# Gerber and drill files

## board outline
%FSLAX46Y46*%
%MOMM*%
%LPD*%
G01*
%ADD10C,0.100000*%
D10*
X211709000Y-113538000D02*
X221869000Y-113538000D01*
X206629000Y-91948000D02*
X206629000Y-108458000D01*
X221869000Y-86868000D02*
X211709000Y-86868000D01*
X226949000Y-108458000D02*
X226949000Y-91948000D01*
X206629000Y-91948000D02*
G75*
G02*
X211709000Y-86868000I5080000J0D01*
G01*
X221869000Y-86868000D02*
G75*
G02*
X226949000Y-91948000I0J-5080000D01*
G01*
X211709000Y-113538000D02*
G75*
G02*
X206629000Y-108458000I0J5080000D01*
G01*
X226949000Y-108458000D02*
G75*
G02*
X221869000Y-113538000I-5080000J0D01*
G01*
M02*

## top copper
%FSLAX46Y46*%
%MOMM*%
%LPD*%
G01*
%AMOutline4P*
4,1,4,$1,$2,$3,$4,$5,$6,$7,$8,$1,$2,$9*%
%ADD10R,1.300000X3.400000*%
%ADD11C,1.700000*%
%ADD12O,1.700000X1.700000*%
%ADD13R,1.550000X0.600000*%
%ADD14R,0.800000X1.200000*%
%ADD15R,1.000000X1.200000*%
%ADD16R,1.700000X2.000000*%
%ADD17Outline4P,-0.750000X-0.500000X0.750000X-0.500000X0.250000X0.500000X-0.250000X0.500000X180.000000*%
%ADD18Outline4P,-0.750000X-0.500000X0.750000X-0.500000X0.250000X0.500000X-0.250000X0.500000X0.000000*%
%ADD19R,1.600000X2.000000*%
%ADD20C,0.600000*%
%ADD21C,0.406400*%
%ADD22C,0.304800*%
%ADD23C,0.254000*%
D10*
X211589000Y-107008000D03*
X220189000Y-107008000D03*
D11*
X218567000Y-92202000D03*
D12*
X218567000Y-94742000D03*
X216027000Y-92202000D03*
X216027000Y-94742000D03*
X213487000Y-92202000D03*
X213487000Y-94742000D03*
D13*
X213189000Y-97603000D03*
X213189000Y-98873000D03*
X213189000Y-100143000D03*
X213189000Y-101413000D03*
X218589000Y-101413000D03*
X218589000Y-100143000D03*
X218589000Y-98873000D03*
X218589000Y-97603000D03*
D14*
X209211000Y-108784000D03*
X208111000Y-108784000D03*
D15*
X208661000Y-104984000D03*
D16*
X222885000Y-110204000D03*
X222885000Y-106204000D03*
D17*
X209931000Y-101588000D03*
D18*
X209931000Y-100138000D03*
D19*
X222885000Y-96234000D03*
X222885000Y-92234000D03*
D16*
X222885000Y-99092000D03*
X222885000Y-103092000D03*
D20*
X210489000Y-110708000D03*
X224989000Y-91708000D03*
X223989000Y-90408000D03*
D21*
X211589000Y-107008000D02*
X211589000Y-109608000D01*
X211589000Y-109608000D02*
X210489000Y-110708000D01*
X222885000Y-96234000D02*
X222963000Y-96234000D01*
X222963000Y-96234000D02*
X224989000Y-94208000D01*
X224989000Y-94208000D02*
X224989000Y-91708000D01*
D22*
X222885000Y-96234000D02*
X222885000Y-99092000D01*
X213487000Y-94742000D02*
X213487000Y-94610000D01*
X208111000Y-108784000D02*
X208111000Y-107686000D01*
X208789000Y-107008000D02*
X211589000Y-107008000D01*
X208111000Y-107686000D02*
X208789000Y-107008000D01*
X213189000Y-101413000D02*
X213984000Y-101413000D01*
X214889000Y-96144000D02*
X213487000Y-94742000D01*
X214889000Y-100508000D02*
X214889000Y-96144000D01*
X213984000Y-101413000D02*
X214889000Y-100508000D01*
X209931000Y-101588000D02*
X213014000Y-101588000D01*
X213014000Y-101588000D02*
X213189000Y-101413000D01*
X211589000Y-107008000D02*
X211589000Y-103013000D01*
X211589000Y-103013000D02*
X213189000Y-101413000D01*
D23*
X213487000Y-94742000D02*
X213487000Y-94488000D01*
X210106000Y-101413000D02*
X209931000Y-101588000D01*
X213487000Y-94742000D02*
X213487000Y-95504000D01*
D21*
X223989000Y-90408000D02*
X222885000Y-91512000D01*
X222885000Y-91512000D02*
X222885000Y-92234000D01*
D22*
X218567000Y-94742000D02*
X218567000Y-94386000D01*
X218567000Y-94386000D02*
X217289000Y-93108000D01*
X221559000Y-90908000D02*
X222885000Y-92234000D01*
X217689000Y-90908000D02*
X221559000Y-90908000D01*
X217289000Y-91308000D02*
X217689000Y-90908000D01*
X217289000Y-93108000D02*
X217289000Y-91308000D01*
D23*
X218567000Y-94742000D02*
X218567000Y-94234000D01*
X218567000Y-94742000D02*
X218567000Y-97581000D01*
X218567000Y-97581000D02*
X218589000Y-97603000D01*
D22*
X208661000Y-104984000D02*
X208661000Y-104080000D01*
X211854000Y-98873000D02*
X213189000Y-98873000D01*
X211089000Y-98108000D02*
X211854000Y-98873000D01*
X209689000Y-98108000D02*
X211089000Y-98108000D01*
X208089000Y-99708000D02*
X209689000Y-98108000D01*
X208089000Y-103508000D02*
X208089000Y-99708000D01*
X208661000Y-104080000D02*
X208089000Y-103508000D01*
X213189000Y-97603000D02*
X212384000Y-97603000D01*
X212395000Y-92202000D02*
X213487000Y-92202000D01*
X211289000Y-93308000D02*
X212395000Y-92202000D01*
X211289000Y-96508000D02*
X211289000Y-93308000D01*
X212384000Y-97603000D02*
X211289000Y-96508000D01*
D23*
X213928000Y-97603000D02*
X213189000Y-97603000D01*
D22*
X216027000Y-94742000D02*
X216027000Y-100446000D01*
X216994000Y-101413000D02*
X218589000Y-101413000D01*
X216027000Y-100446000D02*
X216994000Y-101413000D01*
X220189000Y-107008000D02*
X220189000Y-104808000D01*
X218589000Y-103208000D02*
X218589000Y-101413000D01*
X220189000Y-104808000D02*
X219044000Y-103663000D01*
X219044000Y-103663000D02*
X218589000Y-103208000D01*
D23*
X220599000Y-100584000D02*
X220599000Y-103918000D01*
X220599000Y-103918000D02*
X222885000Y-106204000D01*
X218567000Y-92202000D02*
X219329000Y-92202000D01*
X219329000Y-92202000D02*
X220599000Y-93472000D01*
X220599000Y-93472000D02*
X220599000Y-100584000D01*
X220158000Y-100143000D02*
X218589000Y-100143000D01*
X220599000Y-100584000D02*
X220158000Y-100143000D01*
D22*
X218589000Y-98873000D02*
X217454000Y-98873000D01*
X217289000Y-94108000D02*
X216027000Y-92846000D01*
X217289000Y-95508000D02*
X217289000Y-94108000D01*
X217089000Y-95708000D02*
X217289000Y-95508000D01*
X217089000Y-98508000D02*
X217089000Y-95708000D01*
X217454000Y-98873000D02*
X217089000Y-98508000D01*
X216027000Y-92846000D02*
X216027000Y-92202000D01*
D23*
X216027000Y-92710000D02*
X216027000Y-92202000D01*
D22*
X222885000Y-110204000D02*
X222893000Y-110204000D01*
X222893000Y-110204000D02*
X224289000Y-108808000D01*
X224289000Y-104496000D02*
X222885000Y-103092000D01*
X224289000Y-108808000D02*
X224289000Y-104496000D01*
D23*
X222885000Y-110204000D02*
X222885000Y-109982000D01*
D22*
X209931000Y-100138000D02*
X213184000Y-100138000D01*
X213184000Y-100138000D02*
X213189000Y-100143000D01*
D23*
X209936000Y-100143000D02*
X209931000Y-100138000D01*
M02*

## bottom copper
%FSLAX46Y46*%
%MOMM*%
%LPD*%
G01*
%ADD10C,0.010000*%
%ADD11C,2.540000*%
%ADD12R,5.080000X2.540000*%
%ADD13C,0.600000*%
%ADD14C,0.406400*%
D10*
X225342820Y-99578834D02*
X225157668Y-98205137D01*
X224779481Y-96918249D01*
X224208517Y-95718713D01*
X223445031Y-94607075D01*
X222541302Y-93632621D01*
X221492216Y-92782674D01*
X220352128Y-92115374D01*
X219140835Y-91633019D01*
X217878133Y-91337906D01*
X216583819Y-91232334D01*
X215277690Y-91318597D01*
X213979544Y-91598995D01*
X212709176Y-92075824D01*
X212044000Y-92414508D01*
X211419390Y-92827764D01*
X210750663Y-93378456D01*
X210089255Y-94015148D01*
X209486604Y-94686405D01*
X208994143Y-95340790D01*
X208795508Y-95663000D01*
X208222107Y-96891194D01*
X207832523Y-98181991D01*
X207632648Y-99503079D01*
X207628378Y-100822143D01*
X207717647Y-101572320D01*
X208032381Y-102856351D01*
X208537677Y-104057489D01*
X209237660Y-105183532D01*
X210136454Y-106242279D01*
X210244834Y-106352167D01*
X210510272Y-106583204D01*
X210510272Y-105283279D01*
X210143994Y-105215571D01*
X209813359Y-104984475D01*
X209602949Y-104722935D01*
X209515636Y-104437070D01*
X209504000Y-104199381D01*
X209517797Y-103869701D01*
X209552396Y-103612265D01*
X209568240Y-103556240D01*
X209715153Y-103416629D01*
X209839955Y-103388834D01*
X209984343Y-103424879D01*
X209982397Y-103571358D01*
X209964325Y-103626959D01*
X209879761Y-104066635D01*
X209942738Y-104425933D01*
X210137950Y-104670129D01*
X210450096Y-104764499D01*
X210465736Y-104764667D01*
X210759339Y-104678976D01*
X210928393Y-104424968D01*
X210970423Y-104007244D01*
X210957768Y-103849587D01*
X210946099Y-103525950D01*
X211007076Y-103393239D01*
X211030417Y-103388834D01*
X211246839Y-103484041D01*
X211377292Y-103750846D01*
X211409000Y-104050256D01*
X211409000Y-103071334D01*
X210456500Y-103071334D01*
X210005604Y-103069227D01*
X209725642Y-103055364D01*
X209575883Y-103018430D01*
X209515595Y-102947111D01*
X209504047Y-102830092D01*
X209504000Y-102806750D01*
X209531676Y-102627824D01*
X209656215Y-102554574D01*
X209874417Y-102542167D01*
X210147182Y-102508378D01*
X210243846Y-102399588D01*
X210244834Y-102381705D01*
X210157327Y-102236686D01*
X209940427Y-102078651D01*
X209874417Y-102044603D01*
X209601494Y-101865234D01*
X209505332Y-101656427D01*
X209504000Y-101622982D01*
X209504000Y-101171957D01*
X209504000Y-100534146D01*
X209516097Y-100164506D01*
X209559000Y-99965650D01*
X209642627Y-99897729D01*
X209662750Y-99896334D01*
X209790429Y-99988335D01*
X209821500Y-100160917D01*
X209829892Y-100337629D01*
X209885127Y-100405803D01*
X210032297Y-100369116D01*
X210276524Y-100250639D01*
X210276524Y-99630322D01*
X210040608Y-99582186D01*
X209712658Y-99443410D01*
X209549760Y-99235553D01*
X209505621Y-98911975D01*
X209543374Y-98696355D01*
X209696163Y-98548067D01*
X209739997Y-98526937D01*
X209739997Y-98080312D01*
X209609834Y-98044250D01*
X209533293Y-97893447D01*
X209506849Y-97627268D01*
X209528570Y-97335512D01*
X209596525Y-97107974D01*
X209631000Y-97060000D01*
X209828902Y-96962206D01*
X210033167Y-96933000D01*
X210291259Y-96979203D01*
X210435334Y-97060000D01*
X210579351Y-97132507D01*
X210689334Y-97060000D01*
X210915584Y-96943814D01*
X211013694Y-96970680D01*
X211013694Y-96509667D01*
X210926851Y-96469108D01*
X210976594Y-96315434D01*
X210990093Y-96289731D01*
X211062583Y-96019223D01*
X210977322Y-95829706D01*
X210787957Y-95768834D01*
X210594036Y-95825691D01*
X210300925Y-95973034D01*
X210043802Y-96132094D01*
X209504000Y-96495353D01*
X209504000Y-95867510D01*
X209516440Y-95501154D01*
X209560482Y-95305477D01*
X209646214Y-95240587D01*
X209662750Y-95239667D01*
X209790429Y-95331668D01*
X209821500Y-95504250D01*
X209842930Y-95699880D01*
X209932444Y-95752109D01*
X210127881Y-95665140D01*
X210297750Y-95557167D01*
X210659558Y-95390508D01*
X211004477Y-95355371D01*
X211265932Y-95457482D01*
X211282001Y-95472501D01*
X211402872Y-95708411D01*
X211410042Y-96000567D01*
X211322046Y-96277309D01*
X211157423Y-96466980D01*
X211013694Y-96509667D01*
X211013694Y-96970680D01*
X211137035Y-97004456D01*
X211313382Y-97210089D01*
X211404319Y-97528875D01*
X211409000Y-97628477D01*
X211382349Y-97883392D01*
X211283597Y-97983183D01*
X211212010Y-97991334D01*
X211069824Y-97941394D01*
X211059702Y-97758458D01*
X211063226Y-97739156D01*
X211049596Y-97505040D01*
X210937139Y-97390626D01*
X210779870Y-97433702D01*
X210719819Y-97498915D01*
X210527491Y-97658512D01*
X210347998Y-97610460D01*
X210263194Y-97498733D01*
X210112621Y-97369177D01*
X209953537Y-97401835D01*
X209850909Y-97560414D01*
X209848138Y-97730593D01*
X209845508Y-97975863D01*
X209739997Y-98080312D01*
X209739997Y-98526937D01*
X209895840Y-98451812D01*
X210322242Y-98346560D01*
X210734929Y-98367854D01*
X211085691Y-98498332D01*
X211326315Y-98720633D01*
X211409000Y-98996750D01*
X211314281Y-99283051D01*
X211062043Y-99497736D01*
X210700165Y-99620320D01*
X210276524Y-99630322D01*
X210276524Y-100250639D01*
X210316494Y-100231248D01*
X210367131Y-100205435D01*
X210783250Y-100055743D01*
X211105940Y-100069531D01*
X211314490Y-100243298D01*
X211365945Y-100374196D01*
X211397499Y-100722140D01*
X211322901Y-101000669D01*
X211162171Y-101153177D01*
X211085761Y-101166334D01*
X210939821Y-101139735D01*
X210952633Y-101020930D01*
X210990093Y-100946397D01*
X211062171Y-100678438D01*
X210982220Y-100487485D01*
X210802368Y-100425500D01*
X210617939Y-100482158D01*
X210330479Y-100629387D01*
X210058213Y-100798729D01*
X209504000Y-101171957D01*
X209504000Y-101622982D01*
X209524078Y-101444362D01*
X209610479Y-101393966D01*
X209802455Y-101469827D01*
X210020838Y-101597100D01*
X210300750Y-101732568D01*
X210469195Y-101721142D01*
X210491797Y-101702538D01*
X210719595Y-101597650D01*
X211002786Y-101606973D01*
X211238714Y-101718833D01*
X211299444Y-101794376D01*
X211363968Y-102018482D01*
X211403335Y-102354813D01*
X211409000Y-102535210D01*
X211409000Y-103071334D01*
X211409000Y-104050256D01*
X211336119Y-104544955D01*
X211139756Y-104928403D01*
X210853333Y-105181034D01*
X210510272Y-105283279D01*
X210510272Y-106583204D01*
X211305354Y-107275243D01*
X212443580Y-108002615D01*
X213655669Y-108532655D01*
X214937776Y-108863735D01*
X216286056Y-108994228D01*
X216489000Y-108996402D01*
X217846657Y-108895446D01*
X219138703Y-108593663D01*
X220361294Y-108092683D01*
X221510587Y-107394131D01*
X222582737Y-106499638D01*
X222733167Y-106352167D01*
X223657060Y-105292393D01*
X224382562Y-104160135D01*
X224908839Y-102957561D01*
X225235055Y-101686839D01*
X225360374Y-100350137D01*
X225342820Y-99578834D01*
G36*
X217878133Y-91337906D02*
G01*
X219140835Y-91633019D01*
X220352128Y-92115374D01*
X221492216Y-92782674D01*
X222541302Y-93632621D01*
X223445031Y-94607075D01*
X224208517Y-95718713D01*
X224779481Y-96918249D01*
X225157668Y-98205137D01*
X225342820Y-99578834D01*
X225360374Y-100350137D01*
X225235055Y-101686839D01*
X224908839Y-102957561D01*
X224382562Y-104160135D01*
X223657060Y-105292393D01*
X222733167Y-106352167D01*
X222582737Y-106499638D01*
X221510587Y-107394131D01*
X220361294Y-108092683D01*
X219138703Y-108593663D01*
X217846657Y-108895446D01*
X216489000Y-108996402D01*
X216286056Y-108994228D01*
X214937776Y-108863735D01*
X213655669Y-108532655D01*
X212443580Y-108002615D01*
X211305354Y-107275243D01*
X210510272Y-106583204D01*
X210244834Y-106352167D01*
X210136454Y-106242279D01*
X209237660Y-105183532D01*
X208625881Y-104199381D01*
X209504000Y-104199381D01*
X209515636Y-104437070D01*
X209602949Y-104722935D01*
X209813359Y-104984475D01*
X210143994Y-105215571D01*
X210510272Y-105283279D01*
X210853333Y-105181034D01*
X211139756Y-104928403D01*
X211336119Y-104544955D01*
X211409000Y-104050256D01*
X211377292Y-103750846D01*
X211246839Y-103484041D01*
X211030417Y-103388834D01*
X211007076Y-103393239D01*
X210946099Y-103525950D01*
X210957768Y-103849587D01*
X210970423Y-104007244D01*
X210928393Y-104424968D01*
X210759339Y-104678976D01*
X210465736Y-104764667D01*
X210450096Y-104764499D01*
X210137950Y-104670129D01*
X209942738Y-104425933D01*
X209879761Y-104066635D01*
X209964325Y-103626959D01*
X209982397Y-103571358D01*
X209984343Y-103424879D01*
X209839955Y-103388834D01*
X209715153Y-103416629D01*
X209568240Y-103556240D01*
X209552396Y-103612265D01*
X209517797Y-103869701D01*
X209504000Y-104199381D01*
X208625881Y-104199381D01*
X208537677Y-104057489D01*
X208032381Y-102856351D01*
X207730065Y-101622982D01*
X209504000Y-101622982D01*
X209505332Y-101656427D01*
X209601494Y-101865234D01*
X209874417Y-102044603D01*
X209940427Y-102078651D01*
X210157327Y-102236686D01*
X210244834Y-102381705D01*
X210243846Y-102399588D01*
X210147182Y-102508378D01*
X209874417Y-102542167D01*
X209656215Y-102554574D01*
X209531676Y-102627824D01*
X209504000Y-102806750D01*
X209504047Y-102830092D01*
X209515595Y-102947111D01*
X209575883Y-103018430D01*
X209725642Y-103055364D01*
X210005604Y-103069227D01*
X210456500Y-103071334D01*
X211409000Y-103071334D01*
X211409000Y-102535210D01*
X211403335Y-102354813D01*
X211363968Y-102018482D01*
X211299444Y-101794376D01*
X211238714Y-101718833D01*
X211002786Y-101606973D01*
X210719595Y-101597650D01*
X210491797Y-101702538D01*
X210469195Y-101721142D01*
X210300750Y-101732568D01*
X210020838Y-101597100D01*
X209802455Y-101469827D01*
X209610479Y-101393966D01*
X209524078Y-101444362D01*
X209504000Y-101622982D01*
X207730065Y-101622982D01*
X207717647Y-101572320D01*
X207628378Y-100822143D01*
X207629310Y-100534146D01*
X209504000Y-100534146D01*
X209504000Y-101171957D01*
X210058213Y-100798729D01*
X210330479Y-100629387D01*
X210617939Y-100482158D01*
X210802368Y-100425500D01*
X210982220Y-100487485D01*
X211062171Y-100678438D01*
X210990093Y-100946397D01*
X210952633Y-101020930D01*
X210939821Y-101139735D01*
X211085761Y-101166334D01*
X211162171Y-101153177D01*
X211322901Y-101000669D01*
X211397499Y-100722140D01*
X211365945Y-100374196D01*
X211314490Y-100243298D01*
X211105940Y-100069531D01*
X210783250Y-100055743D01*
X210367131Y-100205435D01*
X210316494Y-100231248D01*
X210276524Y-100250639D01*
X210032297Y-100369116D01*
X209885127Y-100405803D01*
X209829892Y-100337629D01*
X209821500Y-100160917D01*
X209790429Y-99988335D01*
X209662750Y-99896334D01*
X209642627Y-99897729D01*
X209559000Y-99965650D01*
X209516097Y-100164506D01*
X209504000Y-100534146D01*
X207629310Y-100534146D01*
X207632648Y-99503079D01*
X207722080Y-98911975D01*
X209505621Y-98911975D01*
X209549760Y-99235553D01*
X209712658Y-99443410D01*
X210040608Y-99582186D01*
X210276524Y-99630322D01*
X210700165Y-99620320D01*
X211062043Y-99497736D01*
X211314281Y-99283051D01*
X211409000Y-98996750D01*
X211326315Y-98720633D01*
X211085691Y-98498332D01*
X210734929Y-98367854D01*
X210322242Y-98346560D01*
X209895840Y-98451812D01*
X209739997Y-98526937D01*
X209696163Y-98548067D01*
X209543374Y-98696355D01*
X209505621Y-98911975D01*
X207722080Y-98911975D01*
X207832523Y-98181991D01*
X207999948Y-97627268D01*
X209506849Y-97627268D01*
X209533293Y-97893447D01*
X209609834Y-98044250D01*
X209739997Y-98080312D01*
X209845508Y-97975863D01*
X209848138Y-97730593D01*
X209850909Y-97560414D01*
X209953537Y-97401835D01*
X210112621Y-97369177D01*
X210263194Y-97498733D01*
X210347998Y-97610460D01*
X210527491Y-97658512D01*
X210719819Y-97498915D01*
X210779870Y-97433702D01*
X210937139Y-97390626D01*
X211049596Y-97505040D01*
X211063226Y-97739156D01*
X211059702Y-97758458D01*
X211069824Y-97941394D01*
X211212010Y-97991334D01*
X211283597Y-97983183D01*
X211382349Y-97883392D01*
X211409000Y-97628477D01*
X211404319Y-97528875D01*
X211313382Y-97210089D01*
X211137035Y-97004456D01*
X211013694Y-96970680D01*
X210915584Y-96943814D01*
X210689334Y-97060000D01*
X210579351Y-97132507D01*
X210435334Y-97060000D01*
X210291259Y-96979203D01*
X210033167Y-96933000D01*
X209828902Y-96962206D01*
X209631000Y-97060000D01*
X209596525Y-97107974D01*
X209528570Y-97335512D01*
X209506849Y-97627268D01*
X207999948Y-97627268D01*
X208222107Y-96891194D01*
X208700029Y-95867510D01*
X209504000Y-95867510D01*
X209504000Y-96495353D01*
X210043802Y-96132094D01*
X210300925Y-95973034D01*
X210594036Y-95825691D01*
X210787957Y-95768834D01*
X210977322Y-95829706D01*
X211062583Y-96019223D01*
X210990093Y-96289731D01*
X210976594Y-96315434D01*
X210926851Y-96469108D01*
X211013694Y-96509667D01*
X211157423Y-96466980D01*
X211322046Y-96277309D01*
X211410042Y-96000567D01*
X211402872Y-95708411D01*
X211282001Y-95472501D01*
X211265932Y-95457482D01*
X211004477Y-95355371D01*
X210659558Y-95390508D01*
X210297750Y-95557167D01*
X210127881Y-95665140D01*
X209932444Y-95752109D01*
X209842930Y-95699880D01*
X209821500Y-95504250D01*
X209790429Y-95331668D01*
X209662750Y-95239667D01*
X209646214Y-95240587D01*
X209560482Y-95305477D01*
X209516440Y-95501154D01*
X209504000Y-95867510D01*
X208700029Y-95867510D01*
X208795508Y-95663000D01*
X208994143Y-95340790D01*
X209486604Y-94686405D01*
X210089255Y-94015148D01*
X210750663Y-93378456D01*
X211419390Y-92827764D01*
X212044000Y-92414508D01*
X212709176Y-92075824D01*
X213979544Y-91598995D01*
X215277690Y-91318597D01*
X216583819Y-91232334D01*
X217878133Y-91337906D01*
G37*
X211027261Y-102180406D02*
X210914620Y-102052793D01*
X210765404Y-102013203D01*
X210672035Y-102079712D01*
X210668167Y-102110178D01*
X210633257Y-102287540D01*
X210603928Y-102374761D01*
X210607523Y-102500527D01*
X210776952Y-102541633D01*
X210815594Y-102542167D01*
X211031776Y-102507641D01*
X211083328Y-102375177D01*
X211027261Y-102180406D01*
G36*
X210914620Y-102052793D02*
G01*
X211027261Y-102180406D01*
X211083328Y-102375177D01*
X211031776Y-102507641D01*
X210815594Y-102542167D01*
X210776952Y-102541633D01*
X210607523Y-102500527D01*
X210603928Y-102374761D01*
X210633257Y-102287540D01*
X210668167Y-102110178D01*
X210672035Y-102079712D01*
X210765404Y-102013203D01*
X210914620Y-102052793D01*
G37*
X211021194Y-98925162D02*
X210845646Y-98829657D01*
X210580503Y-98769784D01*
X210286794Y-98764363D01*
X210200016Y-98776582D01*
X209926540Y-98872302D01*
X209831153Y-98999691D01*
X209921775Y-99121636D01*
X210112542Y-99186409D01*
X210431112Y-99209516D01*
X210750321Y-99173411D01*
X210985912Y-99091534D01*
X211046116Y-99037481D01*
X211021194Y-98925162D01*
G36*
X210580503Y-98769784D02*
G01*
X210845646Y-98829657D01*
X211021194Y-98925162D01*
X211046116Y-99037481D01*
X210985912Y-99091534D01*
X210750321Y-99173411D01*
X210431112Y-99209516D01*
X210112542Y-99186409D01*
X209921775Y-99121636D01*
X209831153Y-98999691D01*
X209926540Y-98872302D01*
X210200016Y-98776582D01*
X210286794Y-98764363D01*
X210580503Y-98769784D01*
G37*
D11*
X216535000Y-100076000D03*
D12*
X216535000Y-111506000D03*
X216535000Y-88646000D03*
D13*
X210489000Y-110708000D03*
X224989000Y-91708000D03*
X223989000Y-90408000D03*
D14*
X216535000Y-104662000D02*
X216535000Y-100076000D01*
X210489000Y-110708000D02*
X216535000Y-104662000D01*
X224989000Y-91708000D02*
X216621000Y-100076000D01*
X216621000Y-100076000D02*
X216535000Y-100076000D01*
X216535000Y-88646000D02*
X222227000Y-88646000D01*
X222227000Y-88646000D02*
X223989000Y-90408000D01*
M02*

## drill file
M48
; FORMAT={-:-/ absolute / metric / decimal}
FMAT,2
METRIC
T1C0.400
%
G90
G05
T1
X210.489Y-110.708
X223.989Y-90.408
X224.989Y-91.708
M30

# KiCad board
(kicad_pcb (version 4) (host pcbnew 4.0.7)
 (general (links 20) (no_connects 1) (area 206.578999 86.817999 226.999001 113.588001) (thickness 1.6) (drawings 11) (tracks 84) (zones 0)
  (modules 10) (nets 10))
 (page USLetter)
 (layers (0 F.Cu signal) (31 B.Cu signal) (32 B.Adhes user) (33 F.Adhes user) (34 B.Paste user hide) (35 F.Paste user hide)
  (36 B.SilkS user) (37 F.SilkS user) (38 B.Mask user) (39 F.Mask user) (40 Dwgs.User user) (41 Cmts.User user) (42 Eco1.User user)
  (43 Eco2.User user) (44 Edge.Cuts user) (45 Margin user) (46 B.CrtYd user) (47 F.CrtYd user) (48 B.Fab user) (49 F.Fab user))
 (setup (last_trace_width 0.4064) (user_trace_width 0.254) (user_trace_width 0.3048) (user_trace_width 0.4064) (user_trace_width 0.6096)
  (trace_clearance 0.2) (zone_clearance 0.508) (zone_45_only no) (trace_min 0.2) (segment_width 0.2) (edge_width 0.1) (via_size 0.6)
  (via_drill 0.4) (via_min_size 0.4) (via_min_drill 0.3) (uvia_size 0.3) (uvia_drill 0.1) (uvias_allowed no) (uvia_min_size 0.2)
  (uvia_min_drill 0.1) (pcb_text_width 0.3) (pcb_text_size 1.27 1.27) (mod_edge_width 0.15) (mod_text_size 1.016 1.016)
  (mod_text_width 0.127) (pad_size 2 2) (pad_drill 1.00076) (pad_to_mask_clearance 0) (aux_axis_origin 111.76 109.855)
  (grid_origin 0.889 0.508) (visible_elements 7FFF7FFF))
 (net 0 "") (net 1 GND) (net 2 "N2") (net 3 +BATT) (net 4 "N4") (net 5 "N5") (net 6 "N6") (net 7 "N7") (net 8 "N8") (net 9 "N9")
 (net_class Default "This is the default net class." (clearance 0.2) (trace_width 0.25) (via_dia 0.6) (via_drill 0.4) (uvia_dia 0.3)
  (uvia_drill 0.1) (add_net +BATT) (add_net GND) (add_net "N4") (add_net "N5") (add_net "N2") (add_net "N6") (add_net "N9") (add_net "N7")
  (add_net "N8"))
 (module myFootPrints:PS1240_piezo (layer F.Cu) (at 215.889 107.008)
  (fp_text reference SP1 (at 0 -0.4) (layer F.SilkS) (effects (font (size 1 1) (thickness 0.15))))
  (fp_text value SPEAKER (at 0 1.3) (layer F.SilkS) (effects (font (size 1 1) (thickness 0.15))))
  (pad 1 smd rect (at -4.3 0) (size 1.3 3.4) (layers F.Cu F.Paste F.Mask) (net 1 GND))
  (pad 2 smd rect (at 4.3 0) (size 1.3 3.4) (layers F.Cu F.Paste F.Mask) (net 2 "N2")))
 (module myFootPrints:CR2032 (layer B.Cu) (at 216.489 100.108 90)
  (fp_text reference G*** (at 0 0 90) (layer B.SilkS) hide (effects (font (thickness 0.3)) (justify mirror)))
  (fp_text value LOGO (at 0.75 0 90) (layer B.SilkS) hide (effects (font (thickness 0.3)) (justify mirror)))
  (fp_poly
   (pts (xy 0.529166 8.85382) (xy 1.902863 8.668668) (xy 3.189751 8.290481) (xy 4.389287 7.719517) (xy 5.500925 6.956031)
    (xy 6.475379 6.052302) (xy 7.325326 5.003216) (xy 7.992626 3.863128) (xy 8.474981 2.651835) (xy 8.770094 1.389133)
    (xy 8.875666 0.094819) (xy 8.789403 -1.21131) (xy 8.509005 -2.509456) (xy 8.032176 -3.779824) (xy 7.693492 -4.445)
    (xy 7.280236 -5.06961) (xy 6.729544 -5.738337) (xy 6.092852 -6.399745) (xy 5.421595 -7.002396) (xy 4.76721 -7.494857)
    (xy 4.445 -7.693492) (xy 3.216806 -8.266893) (xy 1.926009 -8.656477) (xy 0.604921 -8.856352) (xy -0.714143 -8.860622)
    (xy -1.46432 -8.771353) (xy -2.748351 -8.456619) (xy -3.949489 -7.951323) (xy -5.075532 -7.25134) (xy -6.134279 -6.352546)
    (xy -6.244167 -6.244166) (xy -6.475204 -5.978728) (xy -5.175279 -5.978728) (xy -5.107571 -6.345006) (xy -4.876475 -6.675641)
    (xy -4.614935 -6.886051) (xy -4.32907 -6.973364) (xy -4.091381 -6.985) (xy -3.761701 -6.971203) (xy -3.504265 -6.936604)
    (xy -3.44824 -6.92076) (xy -3.308629 -6.773847) (xy -3.280834 -6.649045) (xy -3.316879 -6.504657) (xy -3.463358 -6.506603)
    (xy -3.518959 -6.524675) (xy -3.958635 -6.609239) (xy -4.317933 -6.546262) (xy -4.562129 -6.35105) (xy -4.656499 -6.038904)
    (xy -4.656667 -6.023264) (xy -4.570976 -5.729661) (xy -4.316968 -5.560607) (xy -3.899244 -5.518577) (xy -3.741587 -5.531232)
    (xy -3.41795 -5.542901) (xy -3.285239 -5.481924) (xy -3.280834 -5.458583) (xy -3.376041 -5.242161) (xy -3.642846 -5.111708)
    (xy -3.942256 -5.08) (xy -2.963334 -5.08) (xy -2.963334 -6.0325) (xy -2.961227 -6.483396) (xy -2.947364 -6.763358)
    (xy -2.91043 -6.913117) (xy -2.839111 -6.973405) (xy -2.722092 -6.984953) (xy -2.69875 -6.985) (xy -2.519824 -6.957324)
    (xy -2.446574 -6.832785) (xy -2.434167 -6.614583) (xy -2.400378 -6.341818) (xy -2.291588 -6.245154) (xy -2.273705 -6.244166)
    (xy -2.128686 -6.331673) (xy -1.970651 -6.548573) (xy -1.936603 -6.614583) (xy -1.757234 -6.887506) (xy -1.548427 -6.983668)
    (xy -1.514982 -6.985) (xy -1.063957 -6.985) (xy -0.426146 -6.985) (xy -0.056506 -6.972903) (xy 0.14235 -6.93) (xy 0.210271 -6.846373)
    (xy 0.211666 -6.82625) (xy 0.119665 -6.698571) (xy -0.052917 -6.6675) (xy -0.229629 -6.659108) (xy -0.297803 -6.603873)
    (xy -0.261116 -6.456703) (xy -0.142639 -6.212476) (xy 0.477678 -6.212476) (xy 0.525814 -6.448392) (xy 0.66459 -6.776342)
    (xy 0.872447 -6.93924) (xy 1.196025 -6.983379) (xy 1.411645 -6.945626) (xy 1.559933 -6.792837) (xy 1.581063 -6.749003)
    (xy 2.027688 -6.749003) (xy 2.06375 -6.879166) (xy 2.214553 -6.955707) (xy 2.480732 -6.982151) (xy 2.772488 -6.96043)
    (xy 3.000026 -6.892475) (xy 3.048 -6.858) (xy 3.145794 -6.660098) (xy 3.175 -6.455833) (xy 3.128797 -6.197741) (xy 3.048 -6.053666)
    (xy 2.975493 -5.909649) (xy 3.048 -5.799666) (xy 3.164186 -5.573416) (xy 3.13732 -5.475306) (xy 3.598333 -5.475306)
    (xy 3.638892 -5.562149) (xy 3.792566 -5.512406) (xy 3.818269 -5.498907) (xy 4.088777 -5.426417) (xy 4.278294 -5.511678)
    (xy 4.339166 -5.701043) (xy 4.282309 -5.894964) (xy 4.134966 -6.188075) (xy 3.975906 -6.445198) (xy 3.612647 -6.985) (xy 4.24049 -6.985)
    (xy 4.606846 -6.97256) (xy 4.802523 -6.928518) (xy 4.867413 -6.842786) (xy 4.868333 -6.82625) (xy 4.776332 -6.698571)
    (xy 4.60375 -6.6675) (xy 4.40812 -6.64607) (xy 4.355891 -6.556556) (xy 4.44286 -6.361119) (xy 4.550833 -6.19125) (xy 4.717492 -5.829442)
    (xy 4.752629 -5.484523) (xy 4.650518 -5.223068) (xy 4.635499 -5.206999) (xy 4.399589 -5.086128) (xy 4.107433 -5.078958)
    (xy 3.830691 -5.166954) (xy 3.64102 -5.331577) (xy 3.598333 -5.475306) (xy 3.13732 -5.475306) (xy 3.103544 -5.351965)
    (xy 2.897911 -5.175618) (xy 2.579125 -5.084681) (xy 2.479523 -5.08) (xy 2.224608 -5.106651) (xy 2.124817 -5.205403)
    (xy 2.116666 -5.27699) (xy 2.166606 -5.419176) (xy 2.349542 -5.429298) (xy 2.368844 -5.425774) (xy 2.60296 -5.439404)
    (xy 2.717374 -5.551861) (xy 2.674298 -5.70913) (xy 2.609085 -5.769181) (xy 2.449488 -5.961509) (xy 2.49754 -6.141002)
    (xy 2.609267 -6.225806) (xy 2.738823 -6.376379) (xy 2.706165 -6.535463) (xy 2.547586 -6.638091) (xy 2.377407 -6.640862)
    (xy 2.132137 -6.643492) (xy 2.027688 -6.749003) (xy 1.581063 -6.749003) (xy 1.656188 -6.59316) (xy 1.76144 -6.166758)
    (xy 1.740146 -5.754071) (xy 1.609668 -5.403309) (xy 1.387367 -5.162685) (xy 1.11125 -5.08) (xy 0.824949 -5.174719)
    (xy 0.610264 -5.426957) (xy 0.48768 -5.788835) (xy 0.477678 -6.212476) (xy -0.142639 -6.212476) (xy -0.123248 -6.172506)
    (xy -0.097435 -6.121869) (xy 0.052257 -5.70575) (xy 0.038469 -5.38306) (xy -0.135298 -5.17451) (xy -0.266196 -5.123055)
    (xy -0.61414 -5.091501) (xy -0.892669 -5.166099) (xy -1.045177 -5.326829) (xy -1.058334 -5.403239) (xy -1.031735 -5.549179)
    (xy -0.91293 -5.536367) (xy -0.838397 -5.498907) (xy -0.570438 -5.426829) (xy -0.379485 -5.50678) (xy -0.3175 -5.686632)
    (xy -0.374158 -5.871061) (xy -0.521387 -6.158521) (xy -0.690729 -6.430787) (xy -1.063957 -6.985) (xy -1.514982 -6.985)
    (xy -1.336362 -6.964922) (xy -1.285966 -6.878521) (xy -1.361827 -6.686545) (xy -1.4891 -6.468162) (xy -1.624568 -6.18825)
    (xy -1.613142 -6.019805) (xy -1.594538 -5.997203) (xy -1.48965 -5.769405) (xy -1.498973 -5.486214) (xy -1.610833 -5.250286)
    (xy -1.686376 -5.189556) (xy -1.910482 -5.125032) (xy -2.246813 -5.085665) (xy -2.42721 -5.08) (xy -2.963334 -5.08) (xy -3.942256 -5.08)
    (xy -4.436955 -5.152881) (xy -4.820403 -5.349244) (xy -5.073034 -5.635667) (xy -5.175279 -5.978728) (xy -6.475204 -5.978728)
    (xy -7.167243 -5.183646) (xy -7.894615 -4.04542) (xy -8.424655 -2.833331) (xy -8.755735 -1.551224) (xy -8.886228 -0.202944)
    (xy -8.888402 0) (xy -8.787446 1.357657) (xy -8.485663 2.649703) (xy -7.984683 3.872294) (xy -7.286131 5.021587) (xy -6.391638 6.093737)
    (xy -6.244167 6.244167) (xy -5.184393 7.16806) (xy -4.052135 7.893562) (xy -2.849561 8.419839) (xy -1.578839 8.746055)
    (xy -0.242137 8.871374) (xy 0.529166 8.85382))
   (layer B.Cu) (width 0.01))
  (fp_poly
   (pts (xy -2.072406 -5.461739) (xy -1.944793 -5.57438) (xy -1.905203 -5.723596) (xy -1.971712 -5.816965) (xy -2.002178 -5.820833)
    (xy -2.17954 -5.855743) (xy -2.266761 -5.885072) (xy -2.392527 -5.881477) (xy -2.433633 -5.712048) (xy -2.434167 -5.673406)
    (xy -2.399641 -5.457224) (xy -2.267177 -5.405672) (xy -2.072406 -5.461739))
   (layer B.Cu) (width 0.01))
  (fp_poly
   (pts (xy 1.182838 -5.467806) (xy 1.278343 -5.643354) (xy 1.338216 -5.908497) (xy 1.343637 -6.202206) (xy 1.331418 -6.288984)
    (xy 1.235698 -6.56246) (xy 1.108309 -6.657847) (xy 0.986364 -6.567225) (xy 0.921591 -6.376458) (xy 0.898484 -6.057888)
    (xy 0.934589 -5.738679) (xy 1.016466 -5.503088) (xy 1.070519 -5.442884) (xy 1.182838 -5.467806))
   (layer B.Cu) (width 0.01))
  (pad 3 smd circle (at 0 0 90) (size 17.78 17.78) (layers B.Paste B.Mask)))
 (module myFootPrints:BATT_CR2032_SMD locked (layer B.Cu) (at 216.535 100.076 90)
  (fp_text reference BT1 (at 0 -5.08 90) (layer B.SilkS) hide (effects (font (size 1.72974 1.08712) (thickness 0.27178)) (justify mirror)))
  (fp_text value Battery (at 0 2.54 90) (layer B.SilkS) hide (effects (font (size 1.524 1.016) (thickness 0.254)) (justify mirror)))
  (pad 2 smd circle (at 0 0 90) (size 2.54 2.54) (layers B.Cu B.Paste B.Mask) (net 1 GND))
  (pad 1 smd rect (at -11.43 0 90) (size 2.54 5.08) (layers B.Cu B.Paste B.Mask) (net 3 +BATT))
  (pad 1 smd rect (at 11.43 0 90) (size 2.54 5.08) (layers B.Cu B.Paste B.Mask) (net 3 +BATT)))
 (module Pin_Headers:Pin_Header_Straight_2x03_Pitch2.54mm (layer F.Cu) (at 218.567 92.202 270)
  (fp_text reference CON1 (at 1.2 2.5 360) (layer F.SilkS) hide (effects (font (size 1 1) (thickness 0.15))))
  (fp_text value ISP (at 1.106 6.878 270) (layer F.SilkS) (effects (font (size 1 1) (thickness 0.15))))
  (pad 1 smd circle (at 0 0 270) (size 1.7 1.7) (layers F.Cu F.Paste F.Mask) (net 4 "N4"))
  (pad 2 smd oval (at 2.54 0 270) (size 1.7 1.7) (layers F.Cu F.Paste F.Mask) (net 3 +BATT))
  (pad 3 smd oval (at 0 2.54 270) (size 1.7 1.7) (layers F.Cu F.Paste F.Mask) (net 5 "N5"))
  (pad 4 smd oval (at 2.54 2.54 270) (size 1.7 1.7) (layers F.Cu F.Paste F.Mask) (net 2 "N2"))
  (pad 5 smd oval (at 0 5.08 270) (size 1.7 1.7) (layers F.Cu F.Paste F.Mask) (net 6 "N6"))
  (pad 6 smd oval (at 2.54 5.08 270) (size 1.7 1.7) (layers F.Cu F.Paste F.Mask) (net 1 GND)))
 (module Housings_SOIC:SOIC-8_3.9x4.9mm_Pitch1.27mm (layer F.Cu) (at 215.889 99.508)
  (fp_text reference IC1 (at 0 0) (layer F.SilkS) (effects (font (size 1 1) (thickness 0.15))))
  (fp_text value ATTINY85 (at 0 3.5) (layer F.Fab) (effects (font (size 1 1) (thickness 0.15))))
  (pad 1 smd rect (at -2.7 -1.905) (size 1.55 0.6) (layers F.Cu F.Paste F.Mask) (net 6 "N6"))
  (pad 2 smd rect (at -2.7 -0.635) (size 1.55 0.6) (layers F.Cu F.Paste F.Mask) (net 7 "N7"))
  (pad 3 smd rect (at -2.7 0.635) (size 1.55 0.6) (layers F.Cu F.Paste F.Mask) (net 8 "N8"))
  (pad 4 smd rect (at -2.7 1.905) (size 1.55 0.6) (layers F.Cu F.Paste F.Mask) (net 1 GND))
  (pad 5 smd rect (at 2.7 1.905) (size 1.55 0.6) (layers F.Cu F.Paste F.Mask) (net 2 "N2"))
  (pad 6 smd rect (at 2.7 0.635) (size 1.55 0.6) (layers F.Cu F.Paste F.Mask) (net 4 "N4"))
  (pad 7 smd rect (at 2.7 -0.635) (size 1.55 0.6) (layers F.Cu F.Paste F.Mask) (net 5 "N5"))
  (pad 8 smd rect (at 2.7 -1.905) (size 1.55 0.6) (layers F.Cu F.Paste F.Mask) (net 3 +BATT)))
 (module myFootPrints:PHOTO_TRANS (layer F.Cu) (at 208.661 106.934 90)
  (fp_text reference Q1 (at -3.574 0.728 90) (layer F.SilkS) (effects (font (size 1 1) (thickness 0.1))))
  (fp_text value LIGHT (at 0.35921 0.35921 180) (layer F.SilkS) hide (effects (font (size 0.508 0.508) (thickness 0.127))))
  (pad 2 smd rect (at -1.85 0.55 90) (size 1.2 0.8) (layers F.Cu F.Paste F.Mask))
  (pad 1 smd rect (at -1.85 -0.55 90) (size 1.2 0.8) (layers F.Cu F.Paste F.Mask) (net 1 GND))
  (pad 3 connect rect (at 1.95 0 90) (size 1.2 1) (layers F.Cu F.Mask) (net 7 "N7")))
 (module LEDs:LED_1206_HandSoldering (layer F.Cu) (at 222.885 108.204 90)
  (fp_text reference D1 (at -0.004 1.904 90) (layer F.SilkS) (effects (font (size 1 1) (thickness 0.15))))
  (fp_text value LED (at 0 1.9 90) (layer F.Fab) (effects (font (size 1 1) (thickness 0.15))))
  (pad 1 smd rect (at -2 0 90) (size 2 1.7) (layers F.Cu F.Paste F.Mask) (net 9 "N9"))
  (pad 2 smd rect (at 2 0 90) (size 2 1.7) (layers F.Cu F.Paste F.Mask) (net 4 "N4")))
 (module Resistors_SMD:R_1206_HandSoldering (layer F.Cu) (at 209.931 100.838 90)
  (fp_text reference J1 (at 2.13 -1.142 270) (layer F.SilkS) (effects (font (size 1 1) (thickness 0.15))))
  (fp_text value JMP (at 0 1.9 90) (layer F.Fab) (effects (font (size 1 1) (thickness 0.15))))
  (pad 1 smd trapezoid (at -0.75 0 180) (size 1 1) (rect_delta 0 0.5) (layers F.Cu F.Paste F.Mask) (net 1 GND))
  (pad 2 smd trapezoid (at 0.7 0) (size 1 1) (rect_delta 0 0.5) (layers F.Cu F.Paste F.Mask) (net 8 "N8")))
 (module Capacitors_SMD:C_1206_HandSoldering (layer F.Cu) (at 222.885 94.234 90)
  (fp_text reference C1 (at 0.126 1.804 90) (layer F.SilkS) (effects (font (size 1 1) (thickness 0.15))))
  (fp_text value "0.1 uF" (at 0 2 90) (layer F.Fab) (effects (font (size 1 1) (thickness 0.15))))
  (pad 1 smd rect (at -2 0 90) (size 2 1.6) (layers F.Cu F.Paste F.Mask) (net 1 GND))
  (pad 2 smd rect (at 2 0 90) (size 2 1.6) (layers F.Cu F.Paste F.Mask) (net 3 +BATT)))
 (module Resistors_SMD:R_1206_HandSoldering (layer F.Cu) (at 222.885 101.092 270)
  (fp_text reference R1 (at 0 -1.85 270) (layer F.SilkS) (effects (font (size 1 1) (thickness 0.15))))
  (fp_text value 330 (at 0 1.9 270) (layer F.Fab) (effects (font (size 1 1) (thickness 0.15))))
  (pad 1 smd rect (at -2 0 270) (size 2 1.7) (layers F.Cu F.Paste F.Mask) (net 1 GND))
  (pad 2 smd rect (at 2 0 270) (size 2 1.7) (layers F.Cu F.Paste F.Mask) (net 9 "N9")))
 (gr_line (start 211.709 113.538) (end 221.869 113.538) (angle 90) (layer Edge.Cuts) (width 0.1))
 (gr_line (start 206.629 91.948) (end 206.629 108.458) (angle 90) (layer Edge.Cuts) (width 0.1))
 (gr_line (start 221.869 86.868) (end 211.709 86.868) (angle 90) (layer Edge.Cuts) (width 0.1))
 (gr_line (start 226.949 108.458) (end 226.949 91.948) (angle 90) (layer Edge.Cuts) (width 0.1))
 (gr_arc (start 211.709 91.948) (end 206.629 91.948) (angle 90) (layer Edge.Cuts) (width 0.1))
 (gr_arc (start 221.869 91.948) (end 221.869 86.868) (angle 90) (layer Edge.Cuts) (width 0.1))
 (gr_arc (start 211.709 108.458) (end 211.709 113.538) (angle 90) (layer Edge.Cuts) (width 0.1))
 (gr_arc (start 221.869 108.458) (end 226.949 108.458) (angle 90) (layer Edge.Cuts) (width 0.1))
 (segment (start 211.589 107.008) (end 211.589 109.608) (width 0.4064) (layer F.Cu) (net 1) (status 400000))
 (segment (start 216.535 104.662) (end 216.535 100.076) (width 0.4064) (layer B.Cu) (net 1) (status 800000))
 (segment (start 210.489 110.708) (end 216.535 104.662) (width 0.4064) (layer B.Cu) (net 1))
 (via (at 210.489 110.708) (size 0.6) (drill 0.4) (layers F.Cu B.Cu) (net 1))
 (segment (start 211.589 109.608) (end 210.489 110.708) (width 0.4064) (layer F.Cu) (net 1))
 (segment (start 222.885 96.234) (end 222.963 96.234) (width 0.4064) (layer F.Cu) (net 1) (status C00000))
 (segment (start 222.963 96.234) (end 224.989 94.208) (width 0.4064) (layer F.Cu) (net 1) (status 400000))
 (segment (start 224.989 91.708) (end 216.621 100.076) (width 0.4064) (layer B.Cu) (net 1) (status 800000))
 (via (at 224.989 91.708) (size 0.6) (drill 0.4) (layers F.Cu B.Cu) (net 1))
 (segment (start 224.989 94.208) (end 224.989 91.708) (width 0.4064) (layer F.Cu) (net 1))
 (segment (start 216.621 100.076) (end 216.535 100.076) (width 0.4064) (layer B.Cu) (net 1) (status C00000))
 (segment (start 222.885 96.234) (end 222.885 99.092) (width 0.3048) (layer F.Cu) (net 1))
 (segment (start 213.487 94.742) (end 213.487 94.61) (width 0.3048) (layer F.Cu) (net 1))
 (segment (start 208.111 108.784) (end 208.111 107.686) (width 0.3048) (layer F.Cu) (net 1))
 (segment (start 208.789 107.008) (end 211.589 107.008) (width 0.3048) (layer F.Cu) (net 1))
 (segment (start 208.111 107.686) (end 208.789 107.008) (width 0.3048) (layer F.Cu) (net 1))
 (segment (start 213.189 101.413) (end 213.984 101.413) (width 0.3048) (layer F.Cu) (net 1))
 (segment (start 214.889 96.144) (end 213.487 94.742) (width 0.3048) (layer F.Cu) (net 1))
 (segment (start 214.889 100.508) (end 214.889 96.144) (width 0.3048) (layer F.Cu) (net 1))
 (segment (start 213.984 101.413) (end 214.889 100.508) (width 0.3048) (layer F.Cu) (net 1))
 (segment (start 209.931 101.588) (end 213.014 101.588) (width 0.3048) (layer F.Cu) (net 1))
 (segment (start 213.014 101.588) (end 213.189 101.413) (width 0.3048) (layer F.Cu) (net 1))
 (segment (start 211.589 107.008) (end 211.589 103.013) (width 0.3048) (layer F.Cu) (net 1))
 (segment (start 211.589 103.013) (end 213.189 101.413) (width 0.3048) (layer F.Cu) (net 1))
 (segment (start 213.487 94.742) (end 213.487 94.488) (width 0.254) (layer F.Cu) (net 1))
 (segment (start 210.106 101.413) (end 209.931 101.588) (width 0.254) (layer F.Cu) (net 1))
 (segment (start 213.487 94.742) (end 213.487 95.504) (width 0.254) (layer F.Cu) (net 1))
 (segment (start 216.535 88.646) (end 222.227 88.646) (width 0.4064) (layer B.Cu) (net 3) (status 400000))
 (segment (start 223.989 90.408) (end 222.885 91.512) (width 0.4064) (layer F.Cu) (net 3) (status 800000))
 (via (at 223.989 90.408) (size 0.6) (drill 0.4) (layers F.Cu B.Cu) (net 3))
 (segment (start 222.227 88.646) (end 223.989 90.408) (width 0.4064) (layer B.Cu) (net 3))
 (segment (start 222.885 91.512) (end 222.885 92.234) (width 0.4064) (layer F.Cu) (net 3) (status C00000))
 (segment (start 218.567 94.742) (end 218.567 94.386) (width 0.3048) (layer F.Cu) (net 3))
 (segment (start 218.567 94.386) (end 217.289 93.108) (width 0.3048) (layer F.Cu) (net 3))
 (segment (start 221.559 90.908) (end 222.885 92.234) (width 0.3048) (layer F.Cu) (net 3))
 (segment (start 217.689 90.908) (end 221.559 90.908) (width 0.3048) (layer F.Cu) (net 3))
 (segment (start 217.289 91.308) (end 217.689 90.908) (width 0.3048) (layer F.Cu) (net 3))
 (segment (start 217.289 93.108) (end 217.289 91.308) (width 0.3048) (layer F.Cu) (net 3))
 (segment (start 218.567 94.742) (end 218.567 94.234) (width 0.254) (layer F.Cu) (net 3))
 (segment (start 218.567 94.742) (end 218.567 97.581) (width 0.254) (layer F.Cu) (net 3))
 (segment (start 218.567 97.581) (end 218.589 97.603) (width 0.254) (layer F.Cu) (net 3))
 (segment (start 208.661 104.984) (end 208.661 104.08) (width 0.3048) (layer F.Cu) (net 7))
 (segment (start 211.854 98.873) (end 213.189 98.873) (width 0.3048) (layer F.Cu) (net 7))
 (segment (start 211.089 98.108) (end 211.854 98.873) (width 0.3048) (layer F.Cu) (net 7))
 (segment (start 209.689 98.108) (end 211.089 98.108) (width 0.3048) (layer F.Cu) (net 7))
 (segment (start 208.089 99.708) (end 209.689 98.108) (width 0.3048) (layer F.Cu) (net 7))
 (segment (start 208.089 103.508) (end 208.089 99.708) (width 0.3048) (layer F.Cu) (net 7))
 (segment (start 208.661 104.08) (end 208.089 103.508) (width 0.3048) (layer F.Cu) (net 7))
 (segment (start 213.189 97.603) (end 212.384 97.603) (width 0.3048) (layer F.Cu) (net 6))
 (segment (start 212.395 92.202) (end 213.487 92.202) (width 0.3048) (layer F.Cu) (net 6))
 (segment (start 211.289 93.308) (end 212.395 92.202) (width 0.3048) (layer F.Cu) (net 6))
 (segment (start 211.289 96.508) (end 211.289 93.308) (width 0.3048) (layer F.Cu) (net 6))
 (segment (start 212.384 97.603) (end 211.289 96.508) (width 0.3048) (layer F.Cu) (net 6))
 (segment (start 213.928 97.603) (end 213.189 97.603) (width 0.254) (layer F.Cu) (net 6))
 (segment (start 216.027 94.742) (end 216.027 100.446) (width 0.3048) (layer F.Cu) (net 2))
 (segment (start 216.994 101.413) (end 218.589 101.413) (width 0.3048) (layer F.Cu) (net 2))
 (segment (start 216.027 100.446) (end 216.994 101.413) (width 0.3048) (layer F.Cu) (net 2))
 (segment (start 220.189 107.008) (end 220.189 104.808) (width 0.3048) (layer F.Cu) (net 2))
 (segment (start 218.589 103.208) (end 218.589 101.413) (width 0.3048) (layer F.Cu) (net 2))
 (segment (start 220.189 104.808) (end 219.044 103.663) (width 0.3048) (layer F.Cu) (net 2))
 (segment (start 219.044 103.663) (end 218.589 103.208) (width 0.3048) (layer F.Cu) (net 2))
 (segment (start 220.599 100.584) (end 220.599 103.918) (width 0.254) (layer F.Cu) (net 4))
 (segment (start 220.599 103.918) (end 222.885 106.204) (width 0.254) (layer F.Cu) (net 4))
 (segment (start 218.567 92.202) (end 219.329 92.202) (width 0.254) (layer F.Cu) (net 4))
 (segment (start 219.329 92.202) (end 220.599 93.472) (width 0.254) (layer F.Cu) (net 4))
 (segment (start 220.599 93.472) (end 220.599 100.584) (width 0.254) (layer F.Cu) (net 4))
 (segment (start 220.158 100.143) (end 218.589 100.143) (width 0.254) (layer F.Cu) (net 4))
 (segment (start 220.599 100.584) (end 220.158 100.143) (width 0.254) (layer F.Cu) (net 4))
 (segment (start 218.589 98.873) (end 217.454 98.873) (width 0.3048) (layer F.Cu) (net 5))
 (segment (start 217.289 94.108) (end 216.027 92.846) (width 0.3048) (layer F.Cu) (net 5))
 (segment (start 217.289 95.508) (end 217.289 94.108) (width 0.3048) (layer F.Cu) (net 5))
 (segment (start 217.089 95.708) (end 217.289 95.508) (width 0.3048) (layer F.Cu) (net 5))
 (segment (start 217.089 98.508) (end 217.089 95.708) (width 0.3048) (layer F.Cu) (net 5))
 (segment (start 217.454 98.873) (end 217.089 98.508) (width 0.3048) (layer F.Cu) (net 5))
 (segment (start 216.027 92.846) (end 216.027 92.202) (width 0.3048) (layer F.Cu) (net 5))
 (segment (start 216.027 92.71) (end 216.027 92.202) (width 0.254) (layer F.Cu) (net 5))
 (segment (start 222.885 110.204) (end 222.893 110.204) (width 0.3048) (layer F.Cu) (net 9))
 (segment (start 222.893 110.204) (end 224.289 108.808) (width 0.3048) (layer F.Cu) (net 9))
 (segment (start 224.289 104.496) (end 222.885 103.092) (width 0.3048) (layer F.Cu) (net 9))
 (segment (start 224.289 108.808) (end 224.289 104.496) (width 0.3048) (layer F.Cu) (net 9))
 (segment (start 222.885 110.204) (end 222.885 109.982) (width 0.254) (layer F.Cu) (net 9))
 (segment (start 209.931 100.138) (end 213.184 100.138) (width 0.3048) (layer F.Cu) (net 8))
 (segment (start 213.184 100.138) (end 213.189 100.143) (width 0.3048) (layer F.Cu) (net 8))
 (segment (start 209.936 100.143) (end 209.931 100.138) (width 0.254) (layer F.Cu) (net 8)))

